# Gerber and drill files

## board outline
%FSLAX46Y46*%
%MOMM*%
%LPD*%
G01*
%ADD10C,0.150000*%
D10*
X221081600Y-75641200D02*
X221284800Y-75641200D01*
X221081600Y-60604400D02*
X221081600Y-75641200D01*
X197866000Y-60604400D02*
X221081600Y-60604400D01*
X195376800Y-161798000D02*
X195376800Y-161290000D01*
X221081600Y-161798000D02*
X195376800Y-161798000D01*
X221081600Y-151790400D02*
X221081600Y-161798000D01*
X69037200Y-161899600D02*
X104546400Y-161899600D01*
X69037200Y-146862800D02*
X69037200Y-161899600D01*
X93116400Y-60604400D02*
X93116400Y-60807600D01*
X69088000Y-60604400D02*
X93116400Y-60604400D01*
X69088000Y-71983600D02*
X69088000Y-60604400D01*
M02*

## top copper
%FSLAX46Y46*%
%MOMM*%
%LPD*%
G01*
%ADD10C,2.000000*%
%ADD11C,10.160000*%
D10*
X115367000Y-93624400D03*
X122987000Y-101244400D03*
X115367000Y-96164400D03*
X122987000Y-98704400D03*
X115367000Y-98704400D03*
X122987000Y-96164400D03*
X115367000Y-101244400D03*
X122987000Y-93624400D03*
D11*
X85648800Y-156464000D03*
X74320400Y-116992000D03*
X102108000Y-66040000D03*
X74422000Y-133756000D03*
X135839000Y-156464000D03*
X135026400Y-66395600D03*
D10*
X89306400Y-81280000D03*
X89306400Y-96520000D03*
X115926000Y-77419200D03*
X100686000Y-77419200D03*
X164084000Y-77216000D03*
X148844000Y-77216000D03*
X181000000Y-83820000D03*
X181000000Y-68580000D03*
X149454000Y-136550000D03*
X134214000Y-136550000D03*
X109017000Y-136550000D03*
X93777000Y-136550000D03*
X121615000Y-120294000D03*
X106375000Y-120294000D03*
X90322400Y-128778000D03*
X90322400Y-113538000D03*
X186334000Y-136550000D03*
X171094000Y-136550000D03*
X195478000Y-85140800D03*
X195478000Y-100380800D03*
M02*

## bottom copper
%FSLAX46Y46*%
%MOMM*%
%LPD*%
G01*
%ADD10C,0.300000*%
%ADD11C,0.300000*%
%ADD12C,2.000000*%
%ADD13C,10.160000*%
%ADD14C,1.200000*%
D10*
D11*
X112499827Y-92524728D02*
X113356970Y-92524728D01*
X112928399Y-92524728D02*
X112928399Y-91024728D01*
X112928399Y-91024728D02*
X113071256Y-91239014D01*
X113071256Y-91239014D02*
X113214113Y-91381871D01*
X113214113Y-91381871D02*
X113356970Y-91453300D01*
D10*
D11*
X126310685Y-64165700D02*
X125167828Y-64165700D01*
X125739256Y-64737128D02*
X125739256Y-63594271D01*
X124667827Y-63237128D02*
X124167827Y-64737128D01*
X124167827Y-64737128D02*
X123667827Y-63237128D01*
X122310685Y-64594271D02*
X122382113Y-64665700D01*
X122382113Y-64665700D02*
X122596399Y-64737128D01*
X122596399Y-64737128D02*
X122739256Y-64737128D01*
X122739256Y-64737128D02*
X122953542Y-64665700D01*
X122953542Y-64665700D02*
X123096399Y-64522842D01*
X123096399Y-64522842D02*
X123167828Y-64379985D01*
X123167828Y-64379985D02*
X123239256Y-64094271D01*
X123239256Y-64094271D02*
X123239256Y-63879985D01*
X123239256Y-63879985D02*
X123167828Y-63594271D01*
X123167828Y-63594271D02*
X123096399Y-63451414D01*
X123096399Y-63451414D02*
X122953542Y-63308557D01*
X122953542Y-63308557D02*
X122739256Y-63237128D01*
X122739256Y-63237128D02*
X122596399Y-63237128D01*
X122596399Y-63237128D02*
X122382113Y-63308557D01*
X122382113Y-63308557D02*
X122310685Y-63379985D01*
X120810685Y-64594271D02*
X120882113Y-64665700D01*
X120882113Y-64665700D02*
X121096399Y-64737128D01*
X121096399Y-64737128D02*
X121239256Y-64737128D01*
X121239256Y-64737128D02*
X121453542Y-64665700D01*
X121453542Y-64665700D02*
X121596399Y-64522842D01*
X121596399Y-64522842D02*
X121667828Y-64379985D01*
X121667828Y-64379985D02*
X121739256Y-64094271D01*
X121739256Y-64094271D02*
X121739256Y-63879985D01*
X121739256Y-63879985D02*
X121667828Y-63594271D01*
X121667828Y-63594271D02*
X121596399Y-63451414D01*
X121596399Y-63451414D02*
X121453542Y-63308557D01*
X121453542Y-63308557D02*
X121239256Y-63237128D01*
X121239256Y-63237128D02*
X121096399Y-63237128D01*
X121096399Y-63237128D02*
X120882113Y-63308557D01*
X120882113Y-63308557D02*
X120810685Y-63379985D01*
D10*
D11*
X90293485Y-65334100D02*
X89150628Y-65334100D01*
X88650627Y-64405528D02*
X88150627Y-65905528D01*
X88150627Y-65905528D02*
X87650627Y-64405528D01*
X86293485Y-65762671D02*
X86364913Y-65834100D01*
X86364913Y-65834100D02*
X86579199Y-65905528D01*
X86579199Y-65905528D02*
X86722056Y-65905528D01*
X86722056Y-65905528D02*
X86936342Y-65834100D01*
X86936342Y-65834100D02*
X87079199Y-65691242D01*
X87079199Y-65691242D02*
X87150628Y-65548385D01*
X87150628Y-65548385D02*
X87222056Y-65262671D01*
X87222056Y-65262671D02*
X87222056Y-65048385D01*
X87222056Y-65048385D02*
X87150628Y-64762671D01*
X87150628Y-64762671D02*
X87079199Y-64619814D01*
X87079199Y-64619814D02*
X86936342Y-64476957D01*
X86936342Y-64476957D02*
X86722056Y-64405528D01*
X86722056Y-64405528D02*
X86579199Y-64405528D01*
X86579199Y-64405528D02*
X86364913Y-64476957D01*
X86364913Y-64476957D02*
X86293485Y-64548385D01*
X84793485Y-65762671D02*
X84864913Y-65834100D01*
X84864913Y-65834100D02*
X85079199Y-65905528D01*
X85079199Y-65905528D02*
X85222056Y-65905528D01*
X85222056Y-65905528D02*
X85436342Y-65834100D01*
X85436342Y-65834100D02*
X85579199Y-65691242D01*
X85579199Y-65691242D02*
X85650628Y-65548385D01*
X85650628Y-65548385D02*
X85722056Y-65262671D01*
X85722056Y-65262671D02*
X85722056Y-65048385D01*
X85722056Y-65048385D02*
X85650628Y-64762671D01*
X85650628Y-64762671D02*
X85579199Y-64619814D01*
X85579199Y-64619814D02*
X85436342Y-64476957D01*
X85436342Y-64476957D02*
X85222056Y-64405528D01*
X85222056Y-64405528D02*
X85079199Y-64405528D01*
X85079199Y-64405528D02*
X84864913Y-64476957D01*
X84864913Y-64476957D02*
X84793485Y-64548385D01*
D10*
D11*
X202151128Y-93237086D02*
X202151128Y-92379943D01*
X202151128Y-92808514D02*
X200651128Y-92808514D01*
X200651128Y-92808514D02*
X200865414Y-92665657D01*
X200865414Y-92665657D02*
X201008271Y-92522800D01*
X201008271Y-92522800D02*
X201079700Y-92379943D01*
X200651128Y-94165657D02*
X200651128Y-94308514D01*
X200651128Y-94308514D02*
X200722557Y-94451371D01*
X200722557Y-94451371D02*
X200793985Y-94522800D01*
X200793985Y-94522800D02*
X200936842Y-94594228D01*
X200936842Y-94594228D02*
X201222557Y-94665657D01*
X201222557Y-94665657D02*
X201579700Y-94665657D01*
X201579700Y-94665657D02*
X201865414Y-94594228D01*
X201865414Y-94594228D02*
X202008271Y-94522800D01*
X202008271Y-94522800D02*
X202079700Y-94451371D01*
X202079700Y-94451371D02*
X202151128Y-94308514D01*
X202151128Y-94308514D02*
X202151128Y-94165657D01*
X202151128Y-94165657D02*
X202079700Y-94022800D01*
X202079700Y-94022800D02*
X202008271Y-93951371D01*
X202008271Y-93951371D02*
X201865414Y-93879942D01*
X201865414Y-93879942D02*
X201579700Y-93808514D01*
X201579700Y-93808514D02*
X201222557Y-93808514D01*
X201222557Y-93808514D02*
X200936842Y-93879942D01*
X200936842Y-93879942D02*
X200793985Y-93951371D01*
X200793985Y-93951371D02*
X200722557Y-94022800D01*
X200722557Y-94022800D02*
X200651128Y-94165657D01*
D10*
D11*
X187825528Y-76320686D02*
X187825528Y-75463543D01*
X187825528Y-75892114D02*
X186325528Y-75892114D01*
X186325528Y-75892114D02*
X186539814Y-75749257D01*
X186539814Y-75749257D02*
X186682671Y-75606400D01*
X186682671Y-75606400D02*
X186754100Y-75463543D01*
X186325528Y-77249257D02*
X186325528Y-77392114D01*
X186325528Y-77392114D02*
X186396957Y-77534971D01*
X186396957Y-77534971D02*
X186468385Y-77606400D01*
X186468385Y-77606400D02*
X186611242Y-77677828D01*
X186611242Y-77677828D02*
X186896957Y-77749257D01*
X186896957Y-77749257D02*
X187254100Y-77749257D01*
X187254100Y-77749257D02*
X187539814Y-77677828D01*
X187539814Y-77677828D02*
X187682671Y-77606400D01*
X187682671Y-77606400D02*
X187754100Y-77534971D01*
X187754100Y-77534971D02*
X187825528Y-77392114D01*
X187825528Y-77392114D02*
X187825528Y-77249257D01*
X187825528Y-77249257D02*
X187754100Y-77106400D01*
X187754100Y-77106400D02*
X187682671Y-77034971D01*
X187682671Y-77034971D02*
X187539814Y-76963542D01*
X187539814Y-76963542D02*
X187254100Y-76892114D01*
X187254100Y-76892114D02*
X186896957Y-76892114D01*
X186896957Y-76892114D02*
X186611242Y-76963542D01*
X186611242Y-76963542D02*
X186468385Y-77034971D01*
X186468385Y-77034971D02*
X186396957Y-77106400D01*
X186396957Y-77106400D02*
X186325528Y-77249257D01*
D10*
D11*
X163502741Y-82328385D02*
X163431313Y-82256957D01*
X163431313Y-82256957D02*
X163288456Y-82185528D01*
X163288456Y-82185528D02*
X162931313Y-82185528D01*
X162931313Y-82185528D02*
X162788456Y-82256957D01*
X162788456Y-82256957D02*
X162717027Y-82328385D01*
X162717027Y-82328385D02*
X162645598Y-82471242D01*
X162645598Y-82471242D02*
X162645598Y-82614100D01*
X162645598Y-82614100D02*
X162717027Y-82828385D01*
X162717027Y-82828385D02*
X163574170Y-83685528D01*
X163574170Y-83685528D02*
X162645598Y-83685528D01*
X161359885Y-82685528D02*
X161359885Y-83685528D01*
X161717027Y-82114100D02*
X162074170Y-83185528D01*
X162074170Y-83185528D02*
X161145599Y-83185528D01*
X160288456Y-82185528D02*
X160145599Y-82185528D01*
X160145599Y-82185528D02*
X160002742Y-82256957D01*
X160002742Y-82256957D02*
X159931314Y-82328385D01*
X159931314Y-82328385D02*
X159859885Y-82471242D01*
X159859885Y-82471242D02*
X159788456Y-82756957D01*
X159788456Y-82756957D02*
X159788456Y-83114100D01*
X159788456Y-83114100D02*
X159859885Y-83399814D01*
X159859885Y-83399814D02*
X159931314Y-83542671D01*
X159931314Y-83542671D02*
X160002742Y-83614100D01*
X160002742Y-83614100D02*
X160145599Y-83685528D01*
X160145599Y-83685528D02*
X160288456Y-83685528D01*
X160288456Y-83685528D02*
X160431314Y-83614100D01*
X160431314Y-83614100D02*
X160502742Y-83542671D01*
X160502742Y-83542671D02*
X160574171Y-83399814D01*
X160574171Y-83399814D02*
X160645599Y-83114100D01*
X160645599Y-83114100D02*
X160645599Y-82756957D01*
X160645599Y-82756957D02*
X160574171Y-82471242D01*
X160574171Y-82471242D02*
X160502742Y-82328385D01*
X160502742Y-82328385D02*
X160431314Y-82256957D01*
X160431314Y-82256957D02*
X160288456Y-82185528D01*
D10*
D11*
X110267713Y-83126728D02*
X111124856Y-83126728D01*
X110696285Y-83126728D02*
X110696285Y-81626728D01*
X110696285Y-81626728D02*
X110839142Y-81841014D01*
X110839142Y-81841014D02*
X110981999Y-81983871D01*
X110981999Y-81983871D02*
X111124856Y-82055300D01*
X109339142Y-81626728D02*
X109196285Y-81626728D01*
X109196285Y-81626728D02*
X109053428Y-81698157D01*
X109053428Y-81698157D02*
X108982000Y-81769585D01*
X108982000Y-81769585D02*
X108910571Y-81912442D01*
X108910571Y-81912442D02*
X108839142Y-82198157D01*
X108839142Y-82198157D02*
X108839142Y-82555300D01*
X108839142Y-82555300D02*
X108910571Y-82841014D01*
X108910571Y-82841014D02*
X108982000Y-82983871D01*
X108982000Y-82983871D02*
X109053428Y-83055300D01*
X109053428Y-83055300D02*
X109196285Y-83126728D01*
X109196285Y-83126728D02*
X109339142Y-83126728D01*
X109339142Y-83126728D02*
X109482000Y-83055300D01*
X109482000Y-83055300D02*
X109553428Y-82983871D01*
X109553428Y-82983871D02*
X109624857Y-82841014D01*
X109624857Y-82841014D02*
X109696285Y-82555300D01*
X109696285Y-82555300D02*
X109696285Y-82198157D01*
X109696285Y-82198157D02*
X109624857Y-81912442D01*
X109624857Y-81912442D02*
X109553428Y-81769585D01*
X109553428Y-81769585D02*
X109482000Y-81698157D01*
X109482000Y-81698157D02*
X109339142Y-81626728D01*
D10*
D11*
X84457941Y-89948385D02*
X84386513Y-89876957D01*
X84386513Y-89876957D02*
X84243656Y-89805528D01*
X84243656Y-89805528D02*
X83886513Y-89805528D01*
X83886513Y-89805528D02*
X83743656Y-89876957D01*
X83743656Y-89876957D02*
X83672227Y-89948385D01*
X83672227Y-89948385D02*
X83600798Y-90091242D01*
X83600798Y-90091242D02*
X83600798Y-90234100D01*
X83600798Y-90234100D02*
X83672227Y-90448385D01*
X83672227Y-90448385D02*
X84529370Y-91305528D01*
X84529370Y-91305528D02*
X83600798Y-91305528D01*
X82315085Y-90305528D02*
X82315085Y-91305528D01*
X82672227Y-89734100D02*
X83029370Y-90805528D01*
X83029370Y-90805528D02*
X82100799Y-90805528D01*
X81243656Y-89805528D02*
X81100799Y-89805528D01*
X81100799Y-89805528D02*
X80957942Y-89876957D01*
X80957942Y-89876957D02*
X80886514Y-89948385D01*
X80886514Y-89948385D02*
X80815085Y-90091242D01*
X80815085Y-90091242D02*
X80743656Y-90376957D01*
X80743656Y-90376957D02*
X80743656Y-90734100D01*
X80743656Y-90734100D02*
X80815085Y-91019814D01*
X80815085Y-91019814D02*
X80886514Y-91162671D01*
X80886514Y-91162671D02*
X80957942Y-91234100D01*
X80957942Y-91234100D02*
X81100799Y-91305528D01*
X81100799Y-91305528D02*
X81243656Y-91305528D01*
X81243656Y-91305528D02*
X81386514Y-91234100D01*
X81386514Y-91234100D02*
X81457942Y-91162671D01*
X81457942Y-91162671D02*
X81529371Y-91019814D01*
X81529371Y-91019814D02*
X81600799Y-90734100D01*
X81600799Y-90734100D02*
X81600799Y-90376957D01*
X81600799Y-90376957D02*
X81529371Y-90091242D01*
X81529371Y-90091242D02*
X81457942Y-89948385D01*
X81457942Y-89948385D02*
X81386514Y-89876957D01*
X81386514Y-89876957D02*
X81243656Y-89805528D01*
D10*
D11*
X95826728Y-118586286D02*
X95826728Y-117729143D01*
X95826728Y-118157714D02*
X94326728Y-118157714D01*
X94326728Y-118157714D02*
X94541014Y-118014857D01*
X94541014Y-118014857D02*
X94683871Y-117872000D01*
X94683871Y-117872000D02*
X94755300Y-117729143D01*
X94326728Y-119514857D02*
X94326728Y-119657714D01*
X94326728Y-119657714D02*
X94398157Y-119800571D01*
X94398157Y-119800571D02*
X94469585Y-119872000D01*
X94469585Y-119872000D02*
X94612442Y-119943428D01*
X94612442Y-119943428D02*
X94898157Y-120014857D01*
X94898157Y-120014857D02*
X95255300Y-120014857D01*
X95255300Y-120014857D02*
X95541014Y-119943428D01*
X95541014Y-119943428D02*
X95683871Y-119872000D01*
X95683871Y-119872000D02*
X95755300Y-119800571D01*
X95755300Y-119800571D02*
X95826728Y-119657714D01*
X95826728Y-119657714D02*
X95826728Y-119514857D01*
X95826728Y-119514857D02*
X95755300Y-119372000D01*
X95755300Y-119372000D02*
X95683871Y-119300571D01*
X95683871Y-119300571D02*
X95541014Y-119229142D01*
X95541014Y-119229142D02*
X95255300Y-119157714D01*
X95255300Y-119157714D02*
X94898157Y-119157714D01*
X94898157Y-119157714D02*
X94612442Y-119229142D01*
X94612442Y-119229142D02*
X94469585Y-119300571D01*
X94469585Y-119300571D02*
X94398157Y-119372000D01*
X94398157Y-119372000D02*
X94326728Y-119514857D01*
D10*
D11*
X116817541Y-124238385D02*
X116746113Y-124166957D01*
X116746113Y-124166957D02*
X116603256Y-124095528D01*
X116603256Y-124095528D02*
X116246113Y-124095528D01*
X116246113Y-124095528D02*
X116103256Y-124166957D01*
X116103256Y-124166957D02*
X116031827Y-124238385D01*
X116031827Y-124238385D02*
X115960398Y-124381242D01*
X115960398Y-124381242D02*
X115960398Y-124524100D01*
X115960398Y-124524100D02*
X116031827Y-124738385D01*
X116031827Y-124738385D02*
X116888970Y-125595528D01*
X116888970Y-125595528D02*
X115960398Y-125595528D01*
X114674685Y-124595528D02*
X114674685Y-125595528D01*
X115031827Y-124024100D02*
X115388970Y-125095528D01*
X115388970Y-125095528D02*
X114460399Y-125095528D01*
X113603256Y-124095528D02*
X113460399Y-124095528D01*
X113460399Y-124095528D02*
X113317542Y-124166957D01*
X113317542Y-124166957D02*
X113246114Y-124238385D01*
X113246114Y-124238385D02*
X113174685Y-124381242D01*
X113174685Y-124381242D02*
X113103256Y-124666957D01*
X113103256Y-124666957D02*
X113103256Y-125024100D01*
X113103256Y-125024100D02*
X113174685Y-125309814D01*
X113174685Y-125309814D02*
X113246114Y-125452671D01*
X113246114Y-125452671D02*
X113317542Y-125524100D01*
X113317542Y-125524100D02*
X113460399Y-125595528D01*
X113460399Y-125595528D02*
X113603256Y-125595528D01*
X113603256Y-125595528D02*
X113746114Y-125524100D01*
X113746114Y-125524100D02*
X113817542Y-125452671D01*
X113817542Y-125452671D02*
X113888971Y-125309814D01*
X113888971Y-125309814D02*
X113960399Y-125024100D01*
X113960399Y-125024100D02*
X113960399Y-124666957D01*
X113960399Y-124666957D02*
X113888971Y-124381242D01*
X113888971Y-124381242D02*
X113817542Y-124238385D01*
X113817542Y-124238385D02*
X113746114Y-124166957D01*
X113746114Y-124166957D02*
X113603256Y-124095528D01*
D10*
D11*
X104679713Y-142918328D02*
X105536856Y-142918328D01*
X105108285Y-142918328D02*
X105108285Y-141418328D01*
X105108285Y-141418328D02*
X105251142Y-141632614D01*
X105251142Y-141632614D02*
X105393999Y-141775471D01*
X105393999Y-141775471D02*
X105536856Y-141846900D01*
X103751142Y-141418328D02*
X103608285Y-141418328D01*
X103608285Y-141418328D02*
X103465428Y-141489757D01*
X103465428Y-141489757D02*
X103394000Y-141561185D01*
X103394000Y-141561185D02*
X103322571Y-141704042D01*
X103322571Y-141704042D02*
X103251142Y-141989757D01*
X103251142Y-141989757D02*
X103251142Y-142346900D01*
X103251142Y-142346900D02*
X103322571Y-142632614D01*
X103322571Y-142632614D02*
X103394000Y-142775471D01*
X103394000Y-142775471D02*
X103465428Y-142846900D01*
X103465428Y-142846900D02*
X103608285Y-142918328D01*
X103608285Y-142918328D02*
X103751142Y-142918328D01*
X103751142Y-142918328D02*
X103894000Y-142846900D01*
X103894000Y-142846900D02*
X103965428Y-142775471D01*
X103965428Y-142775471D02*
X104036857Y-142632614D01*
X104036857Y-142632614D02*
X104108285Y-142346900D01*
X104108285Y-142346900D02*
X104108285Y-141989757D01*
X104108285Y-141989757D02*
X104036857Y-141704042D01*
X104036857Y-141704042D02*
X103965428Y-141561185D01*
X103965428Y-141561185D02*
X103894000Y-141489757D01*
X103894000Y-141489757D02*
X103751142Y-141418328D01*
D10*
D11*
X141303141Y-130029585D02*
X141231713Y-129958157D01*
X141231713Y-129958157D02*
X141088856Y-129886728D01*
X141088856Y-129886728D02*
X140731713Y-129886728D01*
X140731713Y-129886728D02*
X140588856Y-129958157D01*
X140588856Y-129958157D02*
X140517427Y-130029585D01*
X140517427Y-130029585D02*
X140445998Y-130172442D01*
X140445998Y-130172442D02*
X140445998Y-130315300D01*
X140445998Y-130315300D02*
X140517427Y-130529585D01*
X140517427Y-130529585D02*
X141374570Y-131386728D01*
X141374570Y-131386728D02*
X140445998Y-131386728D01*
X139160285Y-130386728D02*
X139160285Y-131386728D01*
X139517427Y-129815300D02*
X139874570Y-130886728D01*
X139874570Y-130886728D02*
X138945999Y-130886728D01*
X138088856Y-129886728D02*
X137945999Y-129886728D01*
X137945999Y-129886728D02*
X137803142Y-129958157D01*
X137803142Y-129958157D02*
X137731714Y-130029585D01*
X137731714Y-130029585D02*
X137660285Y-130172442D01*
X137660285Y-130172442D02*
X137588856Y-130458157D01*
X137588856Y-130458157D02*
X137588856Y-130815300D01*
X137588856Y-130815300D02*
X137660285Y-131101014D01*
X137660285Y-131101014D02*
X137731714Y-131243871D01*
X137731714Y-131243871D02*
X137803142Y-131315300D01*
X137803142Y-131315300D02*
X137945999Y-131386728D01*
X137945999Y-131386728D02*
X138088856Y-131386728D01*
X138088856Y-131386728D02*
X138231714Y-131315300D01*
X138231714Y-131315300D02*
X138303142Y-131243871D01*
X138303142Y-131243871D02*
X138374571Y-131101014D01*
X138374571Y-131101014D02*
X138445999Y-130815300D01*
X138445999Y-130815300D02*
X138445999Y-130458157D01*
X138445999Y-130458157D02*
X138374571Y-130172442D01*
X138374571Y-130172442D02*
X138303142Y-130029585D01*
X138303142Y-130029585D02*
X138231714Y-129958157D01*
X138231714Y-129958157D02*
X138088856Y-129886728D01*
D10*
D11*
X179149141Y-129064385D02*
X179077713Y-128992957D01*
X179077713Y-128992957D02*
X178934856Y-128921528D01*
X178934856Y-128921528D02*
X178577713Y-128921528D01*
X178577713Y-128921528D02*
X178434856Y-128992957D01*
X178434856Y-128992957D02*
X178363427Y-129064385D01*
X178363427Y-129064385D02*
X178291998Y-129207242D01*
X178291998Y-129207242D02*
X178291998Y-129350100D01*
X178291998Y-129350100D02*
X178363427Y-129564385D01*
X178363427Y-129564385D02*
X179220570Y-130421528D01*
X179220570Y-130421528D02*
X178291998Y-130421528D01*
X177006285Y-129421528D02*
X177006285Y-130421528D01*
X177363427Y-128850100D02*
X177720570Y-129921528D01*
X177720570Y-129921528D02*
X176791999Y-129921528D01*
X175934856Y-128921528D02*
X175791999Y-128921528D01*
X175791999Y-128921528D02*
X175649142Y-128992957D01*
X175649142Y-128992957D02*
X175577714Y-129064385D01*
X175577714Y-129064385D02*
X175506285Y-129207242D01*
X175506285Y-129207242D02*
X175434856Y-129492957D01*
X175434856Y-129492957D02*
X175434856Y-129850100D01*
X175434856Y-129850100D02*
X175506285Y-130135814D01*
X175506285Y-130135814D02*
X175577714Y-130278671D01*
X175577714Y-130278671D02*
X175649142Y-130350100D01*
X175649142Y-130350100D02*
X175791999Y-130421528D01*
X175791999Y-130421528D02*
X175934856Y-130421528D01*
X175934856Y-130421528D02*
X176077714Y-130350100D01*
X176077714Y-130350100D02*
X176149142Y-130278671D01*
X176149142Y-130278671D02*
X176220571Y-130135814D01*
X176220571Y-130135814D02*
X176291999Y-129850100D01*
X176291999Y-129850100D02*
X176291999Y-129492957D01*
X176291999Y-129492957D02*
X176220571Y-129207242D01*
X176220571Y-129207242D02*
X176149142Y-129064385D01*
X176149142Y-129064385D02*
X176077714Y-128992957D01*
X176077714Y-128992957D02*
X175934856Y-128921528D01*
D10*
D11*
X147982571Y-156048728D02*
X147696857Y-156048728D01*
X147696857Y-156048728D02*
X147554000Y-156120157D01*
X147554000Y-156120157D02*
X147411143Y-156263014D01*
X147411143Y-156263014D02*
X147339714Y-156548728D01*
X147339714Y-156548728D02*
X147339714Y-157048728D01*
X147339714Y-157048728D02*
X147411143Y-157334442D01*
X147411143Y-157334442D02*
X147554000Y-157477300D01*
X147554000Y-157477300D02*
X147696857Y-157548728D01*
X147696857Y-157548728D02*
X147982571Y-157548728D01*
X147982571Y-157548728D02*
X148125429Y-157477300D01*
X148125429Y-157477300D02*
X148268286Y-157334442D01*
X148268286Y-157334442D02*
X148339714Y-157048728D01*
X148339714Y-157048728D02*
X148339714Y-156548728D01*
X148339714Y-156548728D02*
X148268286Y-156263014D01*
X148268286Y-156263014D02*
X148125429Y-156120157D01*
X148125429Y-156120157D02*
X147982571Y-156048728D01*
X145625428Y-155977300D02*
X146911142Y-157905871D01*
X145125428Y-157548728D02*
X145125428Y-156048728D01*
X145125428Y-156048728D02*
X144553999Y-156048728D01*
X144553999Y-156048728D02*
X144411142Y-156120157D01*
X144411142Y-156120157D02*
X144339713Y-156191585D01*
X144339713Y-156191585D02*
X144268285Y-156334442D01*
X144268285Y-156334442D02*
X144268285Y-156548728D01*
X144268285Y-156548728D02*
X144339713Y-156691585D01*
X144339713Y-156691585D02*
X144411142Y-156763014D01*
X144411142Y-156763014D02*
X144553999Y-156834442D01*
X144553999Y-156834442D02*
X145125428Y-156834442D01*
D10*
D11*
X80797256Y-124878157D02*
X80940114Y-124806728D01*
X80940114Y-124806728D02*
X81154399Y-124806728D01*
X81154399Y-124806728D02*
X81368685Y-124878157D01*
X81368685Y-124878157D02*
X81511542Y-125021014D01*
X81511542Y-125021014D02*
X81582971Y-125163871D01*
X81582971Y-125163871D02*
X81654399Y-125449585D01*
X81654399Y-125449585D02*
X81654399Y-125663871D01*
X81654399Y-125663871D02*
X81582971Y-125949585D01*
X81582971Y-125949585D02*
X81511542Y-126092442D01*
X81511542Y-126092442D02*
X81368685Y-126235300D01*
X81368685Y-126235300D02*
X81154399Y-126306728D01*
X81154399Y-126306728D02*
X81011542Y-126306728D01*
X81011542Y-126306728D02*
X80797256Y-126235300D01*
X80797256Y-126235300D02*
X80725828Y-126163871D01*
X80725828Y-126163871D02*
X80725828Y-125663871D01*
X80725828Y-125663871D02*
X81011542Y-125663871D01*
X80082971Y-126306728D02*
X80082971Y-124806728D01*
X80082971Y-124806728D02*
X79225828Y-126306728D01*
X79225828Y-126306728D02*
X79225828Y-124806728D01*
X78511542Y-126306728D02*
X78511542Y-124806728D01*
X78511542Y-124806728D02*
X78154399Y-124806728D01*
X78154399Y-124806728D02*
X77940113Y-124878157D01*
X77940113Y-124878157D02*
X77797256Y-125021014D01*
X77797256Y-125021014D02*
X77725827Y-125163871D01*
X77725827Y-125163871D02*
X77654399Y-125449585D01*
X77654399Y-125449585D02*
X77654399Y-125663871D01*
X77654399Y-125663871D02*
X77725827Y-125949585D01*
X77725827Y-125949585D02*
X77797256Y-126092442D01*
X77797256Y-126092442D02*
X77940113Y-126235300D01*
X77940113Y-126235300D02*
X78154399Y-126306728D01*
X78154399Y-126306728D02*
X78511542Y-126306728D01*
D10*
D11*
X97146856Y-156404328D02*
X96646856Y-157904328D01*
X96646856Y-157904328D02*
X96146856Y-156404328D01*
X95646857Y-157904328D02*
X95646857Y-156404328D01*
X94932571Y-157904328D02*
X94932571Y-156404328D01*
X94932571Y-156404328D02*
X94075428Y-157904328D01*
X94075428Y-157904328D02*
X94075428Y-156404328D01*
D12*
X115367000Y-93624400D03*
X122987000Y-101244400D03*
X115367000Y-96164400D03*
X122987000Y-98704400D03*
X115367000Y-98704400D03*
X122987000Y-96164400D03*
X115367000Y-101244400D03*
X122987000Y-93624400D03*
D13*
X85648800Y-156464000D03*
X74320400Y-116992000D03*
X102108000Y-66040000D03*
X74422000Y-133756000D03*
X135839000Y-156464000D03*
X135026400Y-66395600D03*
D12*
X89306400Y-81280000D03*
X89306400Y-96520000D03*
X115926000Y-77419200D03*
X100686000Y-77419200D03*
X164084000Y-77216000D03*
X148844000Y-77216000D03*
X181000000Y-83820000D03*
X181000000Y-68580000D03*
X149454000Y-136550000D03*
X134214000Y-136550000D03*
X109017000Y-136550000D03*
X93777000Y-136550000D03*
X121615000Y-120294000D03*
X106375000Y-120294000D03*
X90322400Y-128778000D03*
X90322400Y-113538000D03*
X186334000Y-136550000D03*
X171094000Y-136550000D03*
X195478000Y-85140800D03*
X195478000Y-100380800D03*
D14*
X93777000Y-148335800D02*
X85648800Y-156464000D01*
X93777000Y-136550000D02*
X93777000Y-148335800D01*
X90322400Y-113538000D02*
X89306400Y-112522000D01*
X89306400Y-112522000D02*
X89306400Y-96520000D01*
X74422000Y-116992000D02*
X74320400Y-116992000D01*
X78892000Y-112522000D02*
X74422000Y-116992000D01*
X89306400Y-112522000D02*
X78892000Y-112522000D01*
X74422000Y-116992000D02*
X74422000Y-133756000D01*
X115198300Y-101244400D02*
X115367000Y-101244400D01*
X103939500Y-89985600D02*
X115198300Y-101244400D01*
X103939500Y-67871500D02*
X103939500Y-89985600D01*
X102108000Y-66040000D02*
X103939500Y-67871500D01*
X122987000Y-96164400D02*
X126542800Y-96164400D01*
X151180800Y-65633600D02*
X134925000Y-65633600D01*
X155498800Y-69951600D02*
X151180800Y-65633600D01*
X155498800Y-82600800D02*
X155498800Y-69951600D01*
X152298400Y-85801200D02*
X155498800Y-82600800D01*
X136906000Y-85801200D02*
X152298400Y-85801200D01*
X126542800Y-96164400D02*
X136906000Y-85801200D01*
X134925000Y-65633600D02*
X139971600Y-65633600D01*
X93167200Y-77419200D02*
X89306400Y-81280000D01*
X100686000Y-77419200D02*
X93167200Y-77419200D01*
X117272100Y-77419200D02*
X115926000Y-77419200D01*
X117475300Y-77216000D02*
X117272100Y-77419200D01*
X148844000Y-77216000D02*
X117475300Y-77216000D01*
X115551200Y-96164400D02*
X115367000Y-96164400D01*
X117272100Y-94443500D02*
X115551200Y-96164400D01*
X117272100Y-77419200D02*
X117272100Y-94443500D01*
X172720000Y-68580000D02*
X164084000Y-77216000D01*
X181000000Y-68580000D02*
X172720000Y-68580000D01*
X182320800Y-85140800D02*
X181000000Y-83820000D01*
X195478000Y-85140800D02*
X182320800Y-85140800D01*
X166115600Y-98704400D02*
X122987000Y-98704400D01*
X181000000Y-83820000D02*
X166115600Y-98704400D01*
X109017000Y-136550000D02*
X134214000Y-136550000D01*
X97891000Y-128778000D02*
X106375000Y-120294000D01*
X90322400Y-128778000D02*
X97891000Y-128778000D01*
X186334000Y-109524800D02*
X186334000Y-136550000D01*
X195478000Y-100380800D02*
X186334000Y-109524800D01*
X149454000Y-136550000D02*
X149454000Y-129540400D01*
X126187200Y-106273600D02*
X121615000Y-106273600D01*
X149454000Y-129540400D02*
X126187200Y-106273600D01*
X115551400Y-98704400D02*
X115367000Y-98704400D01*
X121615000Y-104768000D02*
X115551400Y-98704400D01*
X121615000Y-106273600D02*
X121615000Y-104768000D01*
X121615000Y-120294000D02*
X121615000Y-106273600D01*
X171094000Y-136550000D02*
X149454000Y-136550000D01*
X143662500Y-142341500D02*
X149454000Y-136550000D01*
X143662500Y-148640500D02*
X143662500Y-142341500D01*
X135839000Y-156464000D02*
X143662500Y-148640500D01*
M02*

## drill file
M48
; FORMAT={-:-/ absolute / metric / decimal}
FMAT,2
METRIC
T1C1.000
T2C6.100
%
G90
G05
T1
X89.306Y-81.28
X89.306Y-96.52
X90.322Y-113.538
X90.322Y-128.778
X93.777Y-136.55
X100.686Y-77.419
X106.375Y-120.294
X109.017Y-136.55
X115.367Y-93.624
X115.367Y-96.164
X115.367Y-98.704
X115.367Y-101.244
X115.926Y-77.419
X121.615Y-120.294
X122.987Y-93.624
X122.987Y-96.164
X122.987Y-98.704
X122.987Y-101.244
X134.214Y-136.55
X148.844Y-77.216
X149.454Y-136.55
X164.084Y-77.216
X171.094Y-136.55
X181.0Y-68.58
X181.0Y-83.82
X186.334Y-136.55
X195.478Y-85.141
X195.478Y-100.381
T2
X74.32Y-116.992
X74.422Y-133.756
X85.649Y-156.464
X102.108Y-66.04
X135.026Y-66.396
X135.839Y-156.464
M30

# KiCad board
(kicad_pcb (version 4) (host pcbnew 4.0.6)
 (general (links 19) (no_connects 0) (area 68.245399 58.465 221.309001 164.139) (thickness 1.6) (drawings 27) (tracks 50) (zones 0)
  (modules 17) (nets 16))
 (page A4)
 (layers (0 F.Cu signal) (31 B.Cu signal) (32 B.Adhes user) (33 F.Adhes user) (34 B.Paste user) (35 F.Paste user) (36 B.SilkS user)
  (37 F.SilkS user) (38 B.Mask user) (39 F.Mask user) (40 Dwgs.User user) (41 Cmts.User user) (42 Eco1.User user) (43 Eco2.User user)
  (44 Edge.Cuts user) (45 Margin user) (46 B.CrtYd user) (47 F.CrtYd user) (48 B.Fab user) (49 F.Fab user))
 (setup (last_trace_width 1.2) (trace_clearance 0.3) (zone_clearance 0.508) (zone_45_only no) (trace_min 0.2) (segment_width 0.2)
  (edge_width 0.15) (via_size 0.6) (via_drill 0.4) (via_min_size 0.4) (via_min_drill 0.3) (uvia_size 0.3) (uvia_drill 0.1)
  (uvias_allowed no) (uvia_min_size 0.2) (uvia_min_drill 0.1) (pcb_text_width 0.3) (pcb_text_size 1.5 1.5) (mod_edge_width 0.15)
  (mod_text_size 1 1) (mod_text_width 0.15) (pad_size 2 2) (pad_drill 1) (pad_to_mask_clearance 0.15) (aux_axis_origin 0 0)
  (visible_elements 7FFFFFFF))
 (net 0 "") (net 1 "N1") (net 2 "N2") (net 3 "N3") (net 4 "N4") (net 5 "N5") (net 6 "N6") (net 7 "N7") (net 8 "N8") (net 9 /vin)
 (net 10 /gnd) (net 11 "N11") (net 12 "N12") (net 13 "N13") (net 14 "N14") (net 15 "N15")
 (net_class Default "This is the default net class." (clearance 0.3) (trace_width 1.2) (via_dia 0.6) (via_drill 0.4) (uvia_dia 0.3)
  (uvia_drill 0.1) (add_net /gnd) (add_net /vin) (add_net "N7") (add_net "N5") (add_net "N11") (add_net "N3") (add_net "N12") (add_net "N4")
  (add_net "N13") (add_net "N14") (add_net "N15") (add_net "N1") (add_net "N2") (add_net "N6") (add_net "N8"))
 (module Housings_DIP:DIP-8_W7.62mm (layer F.Cu) (at 115.367 93.6244)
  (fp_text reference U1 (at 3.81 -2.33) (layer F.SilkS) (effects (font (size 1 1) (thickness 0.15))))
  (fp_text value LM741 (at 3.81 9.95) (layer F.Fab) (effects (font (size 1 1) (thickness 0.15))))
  (pad 1 thru_hole circle (at 0 0) (size 2 2) (drill 1) (layers *.Cu *.Mask) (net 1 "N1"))
  (pad 5 thru_hole circle (at 7.62 7.62) (size 2 2) (drill 1) (layers *.Cu *.Mask) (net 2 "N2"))
  (pad 2 thru_hole circle (at 0 2.54) (size 2 2) (drill 1) (layers *.Cu *.Mask) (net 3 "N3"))
  (pad 6 thru_hole circle (at 7.62 5.08) (size 2 2) (drill 1) (layers *.Cu *.Mask) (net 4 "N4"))
  (pad 3 thru_hole circle (at 0 5.08) (size 2 2) (drill 1) (layers *.Cu *.Mask) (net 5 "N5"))
  (pad 7 thru_hole circle (at 7.62 2.54) (size 2 2) (drill 1) (layers *.Cu *.Mask) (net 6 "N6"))
  (pad 4 thru_hole circle (at 0 7.62) (size 2 2) (drill 1) (layers *.Cu *.Mask) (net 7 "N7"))
  (pad 8 thru_hole circle (at 7.62 0) (size 2 2) (drill 1) (layers *.Cu *.Mask) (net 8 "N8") (clearance 0.15)))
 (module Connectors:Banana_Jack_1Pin (layer F.Cu) (at 85.6488 156.464 180)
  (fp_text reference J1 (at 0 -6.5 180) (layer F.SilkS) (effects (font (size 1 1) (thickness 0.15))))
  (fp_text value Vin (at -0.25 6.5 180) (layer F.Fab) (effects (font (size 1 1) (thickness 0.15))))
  (pad 1 thru_hole circle (at 0 0 180) (size 10.16 10.16) (drill 6.1) (layers *.Cu *.Mask) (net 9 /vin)))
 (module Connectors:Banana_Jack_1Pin (layer F.Cu) (at 74.3204 116.992)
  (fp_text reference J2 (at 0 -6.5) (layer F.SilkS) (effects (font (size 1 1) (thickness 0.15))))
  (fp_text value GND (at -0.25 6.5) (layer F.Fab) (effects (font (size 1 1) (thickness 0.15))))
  (pad 1 thru_hole circle (at 0 0) (size 10.16 10.16) (drill 6.1) (layers *.Cu *.Mask) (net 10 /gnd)))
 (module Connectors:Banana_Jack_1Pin (layer F.Cu) (at 102.108 66.04 180)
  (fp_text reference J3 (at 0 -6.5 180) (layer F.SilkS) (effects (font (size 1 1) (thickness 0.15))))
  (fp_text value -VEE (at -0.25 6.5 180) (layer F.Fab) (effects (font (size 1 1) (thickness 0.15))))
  (pad 1 thru_hole circle (at 0 0 180) (size 10.16 10.16) (drill 6.1) (layers *.Cu *.Mask) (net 7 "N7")))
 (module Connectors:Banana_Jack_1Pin (layer F.Cu) (at 74.422 133.756)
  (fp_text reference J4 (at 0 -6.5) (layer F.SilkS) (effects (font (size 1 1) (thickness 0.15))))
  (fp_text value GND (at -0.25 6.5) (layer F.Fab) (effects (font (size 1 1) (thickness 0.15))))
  (pad 1 thru_hole circle (at 0 0) (size 10.16 10.16) (drill 6.1) (layers *.Cu *.Mask) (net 10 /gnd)))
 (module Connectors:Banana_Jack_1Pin (layer F.Cu) (at 135.839 156.464)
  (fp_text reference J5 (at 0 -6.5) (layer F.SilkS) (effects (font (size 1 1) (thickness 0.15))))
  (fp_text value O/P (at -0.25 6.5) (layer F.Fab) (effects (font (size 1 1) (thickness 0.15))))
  (pad 1 thru_hole circle (at 0 0) (size 10.16 10.16) (drill 6.1) (layers *.Cu *.Mask) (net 5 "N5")))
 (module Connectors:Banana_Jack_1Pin (layer F.Cu) (at 135.0264 66.3956)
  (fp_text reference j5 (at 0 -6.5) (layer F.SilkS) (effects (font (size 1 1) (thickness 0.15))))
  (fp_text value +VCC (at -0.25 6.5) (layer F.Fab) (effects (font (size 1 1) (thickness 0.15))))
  (pad 1 thru_hole circle (at 0 0) (size 10.16 10.16) (drill 6.1) (layers *.Cu *.Mask) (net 6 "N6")))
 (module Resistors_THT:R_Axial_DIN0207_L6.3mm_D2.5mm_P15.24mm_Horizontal (layer F.Cu) (at 89.3064 81.28 270)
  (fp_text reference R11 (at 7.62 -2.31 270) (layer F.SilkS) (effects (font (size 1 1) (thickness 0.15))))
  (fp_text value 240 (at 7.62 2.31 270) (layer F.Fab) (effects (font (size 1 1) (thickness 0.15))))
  (pad 1 thru_hole circle (at 0 0 270) (size 2 2) (drill 1) (layers *.Cu *.Mask) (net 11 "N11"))
  (pad 2 thru_hole circle (at 15.24 0 270) (size 2 2) (drill 1) (layers *.Cu *.Mask) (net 10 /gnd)))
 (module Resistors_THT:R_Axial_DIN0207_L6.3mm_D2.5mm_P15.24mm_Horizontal (layer F.Cu) (at 115.926 77.4192 180)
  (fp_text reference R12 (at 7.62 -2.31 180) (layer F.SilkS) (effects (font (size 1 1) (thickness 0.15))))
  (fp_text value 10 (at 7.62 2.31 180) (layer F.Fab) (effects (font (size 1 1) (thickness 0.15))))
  (pad 1 thru_hole circle (at 0 0 180) (size 2 2) (drill 1) (layers *.Cu *.Mask) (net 3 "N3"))
  (pad 2 thru_hole circle (at 15.24 0 180) (size 2 2) (drill 1) (layers *.Cu *.Mask) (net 11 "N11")))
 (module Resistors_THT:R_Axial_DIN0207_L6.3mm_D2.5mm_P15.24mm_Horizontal (layer F.Cu) (at 164.084 77.216 180)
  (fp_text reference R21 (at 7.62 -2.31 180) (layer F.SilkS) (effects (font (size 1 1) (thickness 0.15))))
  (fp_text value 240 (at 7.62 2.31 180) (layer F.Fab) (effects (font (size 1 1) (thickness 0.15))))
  (pad 1 thru_hole circle (at 0 0 180) (size 2 2) (drill 1) (layers *.Cu *.Mask) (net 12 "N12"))
  (pad 2 thru_hole circle (at 15.24 0 180) (size 2 2) (drill 1) (layers *.Cu *.Mask) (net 3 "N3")))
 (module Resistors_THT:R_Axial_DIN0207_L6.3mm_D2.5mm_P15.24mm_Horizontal (layer F.Cu) (at 181 83.82 90)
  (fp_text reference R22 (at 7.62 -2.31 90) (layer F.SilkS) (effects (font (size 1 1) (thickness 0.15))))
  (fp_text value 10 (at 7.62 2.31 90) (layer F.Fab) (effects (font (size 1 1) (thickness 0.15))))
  (pad 1 thru_hole circle (at 0 0 90) (size 2 2) (drill 1) (layers *.Cu *.Mask) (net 4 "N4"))
  (pad 2 thru_hole circle (at 15.24 0 90) (size 2 2) (drill 1) (layers *.Cu *.Mask) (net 12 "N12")))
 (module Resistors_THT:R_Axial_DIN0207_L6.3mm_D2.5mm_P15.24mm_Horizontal (layer F.Cu) (at 149.454 136.55 180)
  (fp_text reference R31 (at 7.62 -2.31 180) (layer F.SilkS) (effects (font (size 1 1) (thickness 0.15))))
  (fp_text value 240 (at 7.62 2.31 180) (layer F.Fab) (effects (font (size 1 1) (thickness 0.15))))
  (pad 1 thru_hole circle (at 0 0 180) (size 2 2) (drill 1) (layers *.Cu *.Mask) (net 5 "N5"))
  (pad 2 thru_hole circle (at 15.24 0 180) (size 2 2) (drill 1) (layers *.Cu *.Mask) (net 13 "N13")))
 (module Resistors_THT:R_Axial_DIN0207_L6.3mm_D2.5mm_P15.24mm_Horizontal (layer F.Cu) (at 109.017 136.55 180)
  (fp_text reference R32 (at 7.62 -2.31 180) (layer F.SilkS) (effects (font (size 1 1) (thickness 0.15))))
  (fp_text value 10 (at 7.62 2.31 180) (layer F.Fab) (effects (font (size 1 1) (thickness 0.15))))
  (pad 1 thru_hole circle (at 0 0 180) (size 2 2) (drill 1) (layers *.Cu *.Mask) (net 13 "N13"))
  (pad 2 thru_hole circle (at 15.24 0 180) (size 2 2) (drill 1) (layers *.Cu *.Mask) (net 9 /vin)))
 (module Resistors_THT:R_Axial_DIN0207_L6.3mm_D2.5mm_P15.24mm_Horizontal (layer F.Cu) (at 121.615 120.294 180)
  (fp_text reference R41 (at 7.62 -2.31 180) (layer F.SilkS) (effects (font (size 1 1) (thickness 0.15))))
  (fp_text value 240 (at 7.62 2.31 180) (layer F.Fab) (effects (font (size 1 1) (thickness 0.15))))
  (pad 1 thru_hole circle (at 0 0 180) (size 2 2) (drill 1) (layers *.Cu *.Mask) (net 5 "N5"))
  (pad 2 thru_hole circle (at 15.24 0 180) (size 2 2) (drill 1) (layers *.Cu *.Mask) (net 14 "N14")))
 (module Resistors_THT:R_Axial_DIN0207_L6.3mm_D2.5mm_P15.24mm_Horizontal (layer F.Cu) (at 90.3224 128.778 90)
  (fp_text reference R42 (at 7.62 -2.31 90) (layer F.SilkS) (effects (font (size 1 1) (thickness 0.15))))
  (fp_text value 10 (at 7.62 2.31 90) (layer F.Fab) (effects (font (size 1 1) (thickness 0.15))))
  (pad 1 thru_hole circle (at 0 0 90) (size 2 2) (drill 1) (layers *.Cu *.Mask) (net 14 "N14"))
  (pad 2 thru_hole circle (at 15.24 0 90) (size 2 2) (drill 1) (layers *.Cu *.Mask) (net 10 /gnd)))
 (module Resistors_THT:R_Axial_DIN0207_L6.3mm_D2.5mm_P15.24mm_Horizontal (layer F.Cu) (at 186.334 136.55 180)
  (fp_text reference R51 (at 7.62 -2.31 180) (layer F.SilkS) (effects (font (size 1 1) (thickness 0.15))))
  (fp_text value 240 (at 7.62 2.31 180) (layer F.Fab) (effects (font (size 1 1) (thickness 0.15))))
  (pad 1 thru_hole circle (at 0 0 180) (size 2 2) (drill 1) (layers *.Cu *.Mask) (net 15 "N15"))
  (pad 2 thru_hole circle (at 15.24 0 180) (size 2 2) (drill 1) (layers *.Cu *.Mask) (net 5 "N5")))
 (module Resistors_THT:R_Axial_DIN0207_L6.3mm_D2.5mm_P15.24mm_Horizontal (layer F.Cu) (at 195.478 85.1408 270)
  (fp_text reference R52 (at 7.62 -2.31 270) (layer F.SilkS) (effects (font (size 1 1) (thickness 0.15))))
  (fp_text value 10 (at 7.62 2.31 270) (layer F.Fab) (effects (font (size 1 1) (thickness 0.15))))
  (pad 1 thru_hole circle (at 0 0 270) (size 2 2) (drill 1) (layers *.Cu *.Mask) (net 4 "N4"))
  (pad 2 thru_hole circle (at 15.24 0 270) (size 2 2) (drill 1) (layers *.Cu *.Mask) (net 15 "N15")))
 (gr_line (start 221.0816 75.6412) (end 221.2848 75.6412) (angle 90) (layer Edge.Cuts) (width 0.15))
 (gr_line (start 221.0816 60.6044) (end 221.0816 75.6412) (angle 90) (layer Edge.Cuts) (width 0.15))
 (gr_line (start 197.866 60.6044) (end 221.0816 60.6044) (angle 90) (layer Edge.Cuts) (width 0.15))
 (gr_line (start 195.3768 161.798) (end 195.3768 161.29) (angle 90) (layer Edge.Cuts) (width 0.15))
 (gr_line (start 221.0816 161.798) (end 195.3768 161.798) (angle 90) (layer Edge.Cuts) (width 0.15))
 (gr_line (start 221.0816 151.7904) (end 221.0816 161.798) (angle 90) (layer Edge.Cuts) (width 0.15))
 (gr_line (start 69.0372 161.8996) (end 104.5464 161.8996) (angle 90) (layer Edge.Cuts) (width 0.15))
 (gr_line (start 69.0372 146.8628) (end 69.0372 161.8996) (angle 90) (layer Edge.Cuts) (width 0.15))
 (gr_line (start 93.1164 60.6044) (end 93.1164 60.8076) (angle 90) (layer Edge.Cuts) (width 0.15))
 (gr_line (start 69.088 60.6044) (end 93.1164 60.6044) (angle 90) (layer Edge.Cuts) (width 0.15))
 (gr_line (start 69.088 71.9836) (end 69.088 60.6044) (angle 90) (layer Edge.Cuts) (width 0.15))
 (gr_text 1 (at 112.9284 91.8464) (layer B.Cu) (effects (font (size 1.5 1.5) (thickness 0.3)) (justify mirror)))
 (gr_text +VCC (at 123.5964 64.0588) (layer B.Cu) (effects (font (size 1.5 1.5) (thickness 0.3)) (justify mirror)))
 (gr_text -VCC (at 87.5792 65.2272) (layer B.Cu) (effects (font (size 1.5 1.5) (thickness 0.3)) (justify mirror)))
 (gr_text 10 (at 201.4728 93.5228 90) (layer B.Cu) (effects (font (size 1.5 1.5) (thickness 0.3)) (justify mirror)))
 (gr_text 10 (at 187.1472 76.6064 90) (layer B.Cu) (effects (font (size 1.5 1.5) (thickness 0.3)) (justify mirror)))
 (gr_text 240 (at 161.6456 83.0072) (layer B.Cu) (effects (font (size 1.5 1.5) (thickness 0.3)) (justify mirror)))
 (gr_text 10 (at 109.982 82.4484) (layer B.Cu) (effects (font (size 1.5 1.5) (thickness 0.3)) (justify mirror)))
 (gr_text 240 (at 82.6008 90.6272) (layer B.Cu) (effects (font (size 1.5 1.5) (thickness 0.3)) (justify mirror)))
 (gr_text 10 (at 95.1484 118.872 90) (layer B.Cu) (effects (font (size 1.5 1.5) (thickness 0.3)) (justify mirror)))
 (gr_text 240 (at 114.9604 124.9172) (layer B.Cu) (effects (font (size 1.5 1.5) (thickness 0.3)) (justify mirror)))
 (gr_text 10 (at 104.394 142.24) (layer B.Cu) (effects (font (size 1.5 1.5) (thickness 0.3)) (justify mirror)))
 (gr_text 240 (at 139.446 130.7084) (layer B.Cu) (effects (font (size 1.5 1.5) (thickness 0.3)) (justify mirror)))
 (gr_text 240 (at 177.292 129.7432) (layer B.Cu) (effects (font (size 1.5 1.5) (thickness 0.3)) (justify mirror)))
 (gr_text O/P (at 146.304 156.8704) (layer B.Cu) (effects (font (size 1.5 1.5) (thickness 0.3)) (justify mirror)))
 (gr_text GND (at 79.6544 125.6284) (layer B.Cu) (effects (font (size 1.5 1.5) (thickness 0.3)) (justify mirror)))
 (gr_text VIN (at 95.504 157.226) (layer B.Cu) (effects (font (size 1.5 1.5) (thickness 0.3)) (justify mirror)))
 (segment (start 93.777 148.3358) (end 85.6488 156.464) (width 1.2) (layer B.Cu) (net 9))
 (segment (start 93.777 136.55) (end 93.777 148.3358) (width 1.2) (layer B.Cu) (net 9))
 (segment (start 90.3224 113.538) (end 89.3064 112.522) (width 1.2) (layer B.Cu) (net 10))
 (segment (start 89.3064 112.522) (end 89.3064 96.52) (width 1.2) (layer B.Cu) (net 10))
 (segment (start 74.422 116.992) (end 74.3204 116.992) (width 1.2) (layer B.Cu) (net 10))
 (segment (start 78.892 112.522) (end 74.422 116.992) (width 1.2) (layer B.Cu) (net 10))
 (segment (start 89.3064 112.522) (end 78.892 112.522) (width 1.2) (layer B.Cu) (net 10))
 (segment (start 74.422 116.992) (end 74.422 133.756) (width 1.2) (layer B.Cu) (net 10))
 (segment (start 115.1983 101.2444) (end 115.367 101.2444) (width 1.2) (layer B.Cu) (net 7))
 (segment (start 103.9395 89.9856) (end 115.1983 101.2444) (width 1.2) (layer B.Cu) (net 7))
 (segment (start 103.9395 67.8715) (end 103.9395 89.9856) (width 1.2) (layer B.Cu) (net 7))
 (segment (start 102.108 66.04) (end 103.9395 67.8715) (width 1.2) (layer B.Cu) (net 7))
 (segment (start 122.987 96.1644) (end 126.5428 96.1644) (width 1.2) (layer B.Cu) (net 6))
 (segment (start 151.1808 65.6336) (end 134.925 65.6336) (width 1.2) (layer B.Cu) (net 6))
 (segment (start 155.4988 69.9516) (end 151.1808 65.6336) (width 1.2) (layer B.Cu) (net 6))
 (segment (start 155.4988 82.6008) (end 155.4988 69.9516) (width 1.2) (layer B.Cu) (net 6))
 (segment (start 152.2984 85.8012) (end 155.4988 82.6008) (width 1.2) (layer B.Cu) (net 6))
 (segment (start 136.906 85.8012) (end 152.2984 85.8012) (width 1.2) (layer B.Cu) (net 6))
 (segment (start 126.5428 96.1644) (end 136.906 85.8012) (width 1.2) (layer B.Cu) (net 6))
 (segment (start 134.925 65.6336) (end 139.9716 65.6336) (width 1.2) (layer B.Cu) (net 6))
 (segment (start 93.1672 77.4192) (end 89.3064 81.28) (width 1.2) (layer B.Cu) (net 11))
 (segment (start 100.686 77.4192) (end 93.1672 77.4192) (width 1.2) (layer B.Cu) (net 11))
 (segment (start 117.2721 77.4192) (end 115.926 77.4192) (width 1.2) (layer B.Cu) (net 3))
 (segment (start 117.4753 77.216) (end 117.2721 77.4192) (width 1.2) (layer B.Cu) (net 3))
 (segment (start 148.844 77.216) (end 117.4753 77.216) (width 1.2) (layer B.Cu) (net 3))
 (segment (start 115.5512 96.1644) (end 115.367 96.1644) (width 1.2) (layer B.Cu) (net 3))
 (segment (start 117.2721 94.4435) (end 115.5512 96.1644) (width 1.2) (layer B.Cu) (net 3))
 (segment (start 117.2721 77.4192) (end 117.2721 94.4435) (width 1.2) (layer B.Cu) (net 3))
 (segment (start 172.72 68.58) (end 164.084 77.216) (width 1.2) (layer B.Cu) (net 12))
 (segment (start 181 68.58) (end 172.72 68.58) (width 1.2) (layer B.Cu) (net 12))
 (segment (start 182.3208 85.1408) (end 181 83.82) (width 1.2) (layer B.Cu) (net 4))
 (segment (start 195.478 85.1408) (end 182.3208 85.1408) (width 1.2) (layer B.Cu) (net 4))
 (segment (start 166.1156 98.7044) (end 122.987 98.7044) (width 1.2) (layer B.Cu) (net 4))
 (segment (start 181 83.82) (end 166.1156 98.7044) (width 1.2) (layer B.Cu) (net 4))
 (segment (start 109.017 136.55) (end 134.214 136.55) (width 1.2) (layer B.Cu) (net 13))
 (segment (start 97.891 128.778) (end 106.375 120.294) (width 1.2) (layer B.Cu) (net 14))
 (segment (start 90.3224 128.778) (end 97.891 128.778) (width 1.2) (layer B.Cu) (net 14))
 (segment (start 186.334 109.5248) (end 186.334 136.55) (width 1.2) (layer B.Cu) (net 15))
 (segment (start 195.478 100.3808) (end 186.334 109.5248) (width 1.2) (layer B.Cu) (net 15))
 (segment (start 149.454 136.55) (end 149.454 129.5404) (width 1.2) (layer B.Cu) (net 5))
 (segment (start 126.1872 106.2736) (end 121.615 106.2736) (width 1.2) (layer B.Cu) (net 5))
 (segment (start 149.454 129.5404) (end 126.1872 106.2736) (width 1.2) (layer B.Cu) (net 5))
 (segment (start 115.5514 98.7044) (end 115.367 98.7044) (width 1.2) (layer B.Cu) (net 5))
 (segment (start 121.615 104.768) (end 115.5514 98.7044) (width 1.2) (layer B.Cu) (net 5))
 (segment (start 121.615 106.2736) (end 121.615 104.768) (width 1.2) (layer B.Cu) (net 5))
 (segment (start 121.615 120.294) (end 121.615 106.2736) (width 1.2) (layer B.Cu) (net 5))
 (segment (start 171.094 136.55) (end 149.454 136.55) (width 1.2) (layer B.Cu) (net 5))
 (segment (start 143.6625 142.3415) (end 149.454 136.55) (width 1.2) (layer B.Cu) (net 5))
 (segment (start 143.6625 148.6405) (end 143.6625 142.3415) (width 1.2) (layer B.Cu) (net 5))
 (segment (start 135.839 156.464) (end 143.6625 148.6405) (width 1.2) (layer B.Cu) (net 5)))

